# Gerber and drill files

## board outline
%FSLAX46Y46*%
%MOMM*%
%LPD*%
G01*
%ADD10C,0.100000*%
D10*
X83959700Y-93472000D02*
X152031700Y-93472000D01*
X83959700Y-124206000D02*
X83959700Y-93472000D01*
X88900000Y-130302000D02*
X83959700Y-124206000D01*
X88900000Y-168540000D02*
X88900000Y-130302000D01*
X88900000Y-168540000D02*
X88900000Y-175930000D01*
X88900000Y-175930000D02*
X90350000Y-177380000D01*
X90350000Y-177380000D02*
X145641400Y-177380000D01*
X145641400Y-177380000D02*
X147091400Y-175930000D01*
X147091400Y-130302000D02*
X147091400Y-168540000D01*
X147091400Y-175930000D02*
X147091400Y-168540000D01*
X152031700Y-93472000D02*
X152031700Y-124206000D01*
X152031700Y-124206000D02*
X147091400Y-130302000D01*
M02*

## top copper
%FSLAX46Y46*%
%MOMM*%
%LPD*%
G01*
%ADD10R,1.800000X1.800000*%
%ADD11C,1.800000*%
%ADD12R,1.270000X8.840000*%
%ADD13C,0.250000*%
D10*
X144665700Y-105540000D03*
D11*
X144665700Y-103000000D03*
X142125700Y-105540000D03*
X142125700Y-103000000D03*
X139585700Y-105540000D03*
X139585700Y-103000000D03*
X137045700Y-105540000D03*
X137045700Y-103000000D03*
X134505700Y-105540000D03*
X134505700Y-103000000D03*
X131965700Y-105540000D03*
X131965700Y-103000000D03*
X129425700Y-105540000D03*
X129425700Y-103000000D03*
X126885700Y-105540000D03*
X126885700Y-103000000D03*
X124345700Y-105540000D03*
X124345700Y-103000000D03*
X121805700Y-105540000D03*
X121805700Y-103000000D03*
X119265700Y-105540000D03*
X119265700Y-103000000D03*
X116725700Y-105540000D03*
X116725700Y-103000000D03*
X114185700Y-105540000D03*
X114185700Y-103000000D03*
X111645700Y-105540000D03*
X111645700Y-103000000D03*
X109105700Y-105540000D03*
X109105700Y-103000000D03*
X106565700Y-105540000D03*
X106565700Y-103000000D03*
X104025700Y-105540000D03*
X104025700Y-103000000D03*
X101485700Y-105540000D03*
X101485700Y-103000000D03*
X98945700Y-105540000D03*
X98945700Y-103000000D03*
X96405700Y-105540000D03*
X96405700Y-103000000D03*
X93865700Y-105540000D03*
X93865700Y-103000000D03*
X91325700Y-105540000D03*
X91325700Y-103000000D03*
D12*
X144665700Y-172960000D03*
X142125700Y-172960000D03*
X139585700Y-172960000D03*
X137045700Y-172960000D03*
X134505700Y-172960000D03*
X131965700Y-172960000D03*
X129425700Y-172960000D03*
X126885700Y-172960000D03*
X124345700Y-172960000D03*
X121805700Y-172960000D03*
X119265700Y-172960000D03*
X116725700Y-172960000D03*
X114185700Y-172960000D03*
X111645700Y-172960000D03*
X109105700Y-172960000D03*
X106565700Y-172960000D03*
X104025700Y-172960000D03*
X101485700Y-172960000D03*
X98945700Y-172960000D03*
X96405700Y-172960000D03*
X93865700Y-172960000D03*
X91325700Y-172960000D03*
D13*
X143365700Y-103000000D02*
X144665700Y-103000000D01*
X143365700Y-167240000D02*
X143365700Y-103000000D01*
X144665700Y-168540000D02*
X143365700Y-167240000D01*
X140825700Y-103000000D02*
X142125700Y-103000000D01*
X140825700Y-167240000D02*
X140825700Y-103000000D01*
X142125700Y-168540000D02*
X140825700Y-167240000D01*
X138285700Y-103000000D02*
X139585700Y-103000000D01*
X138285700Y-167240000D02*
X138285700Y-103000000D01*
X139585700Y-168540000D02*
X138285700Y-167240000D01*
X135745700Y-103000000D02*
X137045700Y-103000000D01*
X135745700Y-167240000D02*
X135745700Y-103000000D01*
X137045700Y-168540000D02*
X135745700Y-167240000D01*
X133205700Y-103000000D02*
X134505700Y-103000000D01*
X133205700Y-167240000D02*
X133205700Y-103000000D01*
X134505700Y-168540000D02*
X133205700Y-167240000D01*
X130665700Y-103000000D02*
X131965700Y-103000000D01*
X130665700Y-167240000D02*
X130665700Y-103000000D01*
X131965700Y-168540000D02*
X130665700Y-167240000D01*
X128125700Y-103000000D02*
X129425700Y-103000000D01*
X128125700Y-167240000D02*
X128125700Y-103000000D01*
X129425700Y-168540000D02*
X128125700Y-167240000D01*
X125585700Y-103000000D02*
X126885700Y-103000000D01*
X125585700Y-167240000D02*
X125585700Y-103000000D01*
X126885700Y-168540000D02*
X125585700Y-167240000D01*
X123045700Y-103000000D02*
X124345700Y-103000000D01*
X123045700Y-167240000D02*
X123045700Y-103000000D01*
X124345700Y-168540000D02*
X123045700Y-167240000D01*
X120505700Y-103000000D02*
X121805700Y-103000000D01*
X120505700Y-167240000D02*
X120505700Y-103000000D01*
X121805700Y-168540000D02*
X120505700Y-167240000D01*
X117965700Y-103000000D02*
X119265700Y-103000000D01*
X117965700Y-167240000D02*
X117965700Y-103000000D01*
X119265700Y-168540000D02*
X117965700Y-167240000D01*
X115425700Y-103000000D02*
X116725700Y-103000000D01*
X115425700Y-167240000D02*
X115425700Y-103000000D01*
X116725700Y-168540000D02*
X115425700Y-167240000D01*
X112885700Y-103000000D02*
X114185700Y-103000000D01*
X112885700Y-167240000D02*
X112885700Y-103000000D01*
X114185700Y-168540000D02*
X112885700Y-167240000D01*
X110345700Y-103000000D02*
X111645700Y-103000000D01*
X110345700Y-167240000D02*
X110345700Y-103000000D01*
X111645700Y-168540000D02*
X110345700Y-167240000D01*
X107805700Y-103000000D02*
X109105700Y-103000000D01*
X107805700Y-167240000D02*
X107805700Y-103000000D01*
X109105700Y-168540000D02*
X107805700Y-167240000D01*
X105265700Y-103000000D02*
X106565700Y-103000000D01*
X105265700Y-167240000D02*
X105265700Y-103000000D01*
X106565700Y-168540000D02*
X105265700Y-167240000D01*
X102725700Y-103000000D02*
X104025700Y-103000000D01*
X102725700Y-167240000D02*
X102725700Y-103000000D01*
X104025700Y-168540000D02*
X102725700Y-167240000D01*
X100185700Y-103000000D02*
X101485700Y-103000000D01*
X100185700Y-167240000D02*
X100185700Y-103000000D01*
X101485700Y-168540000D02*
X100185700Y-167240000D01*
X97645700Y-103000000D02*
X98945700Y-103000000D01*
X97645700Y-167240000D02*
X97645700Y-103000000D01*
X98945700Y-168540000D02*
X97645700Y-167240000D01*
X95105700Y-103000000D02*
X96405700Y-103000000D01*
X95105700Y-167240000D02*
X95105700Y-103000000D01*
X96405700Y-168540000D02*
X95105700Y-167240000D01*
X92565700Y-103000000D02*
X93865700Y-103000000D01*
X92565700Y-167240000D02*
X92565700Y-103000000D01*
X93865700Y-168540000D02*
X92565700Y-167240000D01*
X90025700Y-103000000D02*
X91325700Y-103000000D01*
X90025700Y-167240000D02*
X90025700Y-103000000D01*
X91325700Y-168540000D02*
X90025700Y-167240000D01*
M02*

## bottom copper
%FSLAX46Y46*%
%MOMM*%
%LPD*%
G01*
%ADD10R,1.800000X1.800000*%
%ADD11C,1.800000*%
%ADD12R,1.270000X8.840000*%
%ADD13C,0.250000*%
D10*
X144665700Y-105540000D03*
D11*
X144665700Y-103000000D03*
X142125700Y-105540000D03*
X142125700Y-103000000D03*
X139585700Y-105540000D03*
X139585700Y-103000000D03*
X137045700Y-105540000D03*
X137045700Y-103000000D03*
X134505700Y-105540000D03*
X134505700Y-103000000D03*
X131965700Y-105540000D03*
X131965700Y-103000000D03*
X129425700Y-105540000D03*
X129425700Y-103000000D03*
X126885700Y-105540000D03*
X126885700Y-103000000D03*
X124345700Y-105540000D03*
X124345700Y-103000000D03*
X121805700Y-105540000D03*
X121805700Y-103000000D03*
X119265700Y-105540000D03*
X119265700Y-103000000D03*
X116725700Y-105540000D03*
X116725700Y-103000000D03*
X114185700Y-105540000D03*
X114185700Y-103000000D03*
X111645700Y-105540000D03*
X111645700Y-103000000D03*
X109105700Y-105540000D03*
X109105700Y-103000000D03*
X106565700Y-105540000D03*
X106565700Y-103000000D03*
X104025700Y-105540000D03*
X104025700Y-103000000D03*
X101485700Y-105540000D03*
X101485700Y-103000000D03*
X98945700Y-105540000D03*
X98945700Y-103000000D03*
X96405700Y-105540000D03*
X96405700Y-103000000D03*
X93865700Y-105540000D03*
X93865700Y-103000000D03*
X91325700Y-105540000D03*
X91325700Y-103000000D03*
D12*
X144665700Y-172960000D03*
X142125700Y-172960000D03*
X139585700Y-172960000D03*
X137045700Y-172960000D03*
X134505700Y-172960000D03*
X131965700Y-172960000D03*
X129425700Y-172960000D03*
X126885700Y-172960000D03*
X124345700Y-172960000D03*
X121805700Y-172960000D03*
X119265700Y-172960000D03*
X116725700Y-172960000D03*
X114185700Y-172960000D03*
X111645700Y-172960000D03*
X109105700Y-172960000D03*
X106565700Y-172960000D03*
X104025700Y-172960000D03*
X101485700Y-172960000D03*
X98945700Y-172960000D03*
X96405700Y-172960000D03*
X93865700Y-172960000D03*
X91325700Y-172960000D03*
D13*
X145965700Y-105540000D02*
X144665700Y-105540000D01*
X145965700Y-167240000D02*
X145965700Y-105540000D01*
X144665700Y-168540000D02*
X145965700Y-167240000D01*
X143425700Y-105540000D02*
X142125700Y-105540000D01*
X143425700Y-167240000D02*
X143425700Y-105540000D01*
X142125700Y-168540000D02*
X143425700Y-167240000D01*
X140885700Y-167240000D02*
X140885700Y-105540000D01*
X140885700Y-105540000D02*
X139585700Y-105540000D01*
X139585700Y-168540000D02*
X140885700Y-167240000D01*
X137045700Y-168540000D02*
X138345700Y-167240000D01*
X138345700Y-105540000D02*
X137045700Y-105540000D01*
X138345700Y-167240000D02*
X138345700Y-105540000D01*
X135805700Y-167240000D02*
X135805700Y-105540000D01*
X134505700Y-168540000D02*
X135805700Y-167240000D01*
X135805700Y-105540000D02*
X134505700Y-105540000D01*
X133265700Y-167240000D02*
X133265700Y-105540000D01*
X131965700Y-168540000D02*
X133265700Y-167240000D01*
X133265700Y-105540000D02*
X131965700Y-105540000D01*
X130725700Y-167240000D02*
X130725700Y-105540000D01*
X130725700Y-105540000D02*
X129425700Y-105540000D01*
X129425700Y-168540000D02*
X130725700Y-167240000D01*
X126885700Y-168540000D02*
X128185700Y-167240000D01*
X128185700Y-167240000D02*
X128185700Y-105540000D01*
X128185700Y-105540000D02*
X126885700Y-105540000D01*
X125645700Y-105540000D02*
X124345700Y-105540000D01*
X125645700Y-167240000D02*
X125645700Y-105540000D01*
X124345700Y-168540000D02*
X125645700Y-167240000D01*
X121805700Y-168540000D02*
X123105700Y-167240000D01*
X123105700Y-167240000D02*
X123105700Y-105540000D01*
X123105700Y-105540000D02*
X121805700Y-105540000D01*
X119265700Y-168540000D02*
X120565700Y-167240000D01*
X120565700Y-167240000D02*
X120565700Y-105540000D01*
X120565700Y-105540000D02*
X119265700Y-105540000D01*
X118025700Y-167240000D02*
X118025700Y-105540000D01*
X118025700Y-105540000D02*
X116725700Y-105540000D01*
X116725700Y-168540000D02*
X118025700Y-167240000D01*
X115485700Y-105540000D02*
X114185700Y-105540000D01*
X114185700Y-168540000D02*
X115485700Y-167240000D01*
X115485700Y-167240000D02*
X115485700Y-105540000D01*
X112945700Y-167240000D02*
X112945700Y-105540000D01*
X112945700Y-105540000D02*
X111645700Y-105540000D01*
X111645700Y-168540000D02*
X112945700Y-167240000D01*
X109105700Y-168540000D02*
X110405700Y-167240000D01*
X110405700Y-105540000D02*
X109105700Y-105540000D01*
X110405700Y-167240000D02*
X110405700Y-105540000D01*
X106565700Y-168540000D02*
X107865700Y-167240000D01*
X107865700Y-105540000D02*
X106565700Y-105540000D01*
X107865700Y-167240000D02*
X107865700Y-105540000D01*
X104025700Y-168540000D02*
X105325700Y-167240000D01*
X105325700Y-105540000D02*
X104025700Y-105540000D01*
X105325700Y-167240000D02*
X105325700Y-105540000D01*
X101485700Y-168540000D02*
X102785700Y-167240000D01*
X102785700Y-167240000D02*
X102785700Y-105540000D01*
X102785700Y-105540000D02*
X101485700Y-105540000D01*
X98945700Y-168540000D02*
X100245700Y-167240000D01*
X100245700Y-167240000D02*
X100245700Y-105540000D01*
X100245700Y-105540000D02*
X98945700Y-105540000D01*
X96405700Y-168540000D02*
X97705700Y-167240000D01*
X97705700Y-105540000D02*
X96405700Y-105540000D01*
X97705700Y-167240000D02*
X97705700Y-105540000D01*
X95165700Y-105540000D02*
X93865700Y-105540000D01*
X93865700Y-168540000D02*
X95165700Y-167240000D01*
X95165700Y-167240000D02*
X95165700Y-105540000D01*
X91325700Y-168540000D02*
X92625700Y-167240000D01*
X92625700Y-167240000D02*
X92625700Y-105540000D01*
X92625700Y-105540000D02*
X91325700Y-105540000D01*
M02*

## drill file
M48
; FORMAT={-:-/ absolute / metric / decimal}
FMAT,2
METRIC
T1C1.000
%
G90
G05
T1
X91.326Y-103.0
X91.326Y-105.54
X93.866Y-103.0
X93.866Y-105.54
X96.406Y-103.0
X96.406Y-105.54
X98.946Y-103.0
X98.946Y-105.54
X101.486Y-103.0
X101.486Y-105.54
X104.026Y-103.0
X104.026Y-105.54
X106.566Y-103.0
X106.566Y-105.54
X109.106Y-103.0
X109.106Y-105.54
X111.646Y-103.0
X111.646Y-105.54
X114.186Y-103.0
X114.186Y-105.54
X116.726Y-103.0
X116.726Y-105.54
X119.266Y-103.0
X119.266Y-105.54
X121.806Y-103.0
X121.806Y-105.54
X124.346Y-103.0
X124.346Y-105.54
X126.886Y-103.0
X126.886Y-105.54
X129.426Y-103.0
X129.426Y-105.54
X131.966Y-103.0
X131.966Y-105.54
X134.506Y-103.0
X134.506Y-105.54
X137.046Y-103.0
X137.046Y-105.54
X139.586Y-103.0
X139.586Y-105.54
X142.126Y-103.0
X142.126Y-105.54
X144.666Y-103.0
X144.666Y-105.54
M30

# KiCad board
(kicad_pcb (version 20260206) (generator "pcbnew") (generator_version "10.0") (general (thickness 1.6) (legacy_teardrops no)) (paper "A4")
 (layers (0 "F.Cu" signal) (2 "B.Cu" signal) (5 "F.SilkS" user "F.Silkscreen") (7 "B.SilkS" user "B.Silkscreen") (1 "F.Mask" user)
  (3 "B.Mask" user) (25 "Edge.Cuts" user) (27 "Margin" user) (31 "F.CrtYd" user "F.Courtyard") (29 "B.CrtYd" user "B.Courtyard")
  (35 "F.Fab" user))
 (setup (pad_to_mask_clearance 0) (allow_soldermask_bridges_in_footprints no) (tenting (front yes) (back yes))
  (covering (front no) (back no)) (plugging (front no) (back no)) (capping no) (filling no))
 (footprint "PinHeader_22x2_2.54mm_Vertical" (layer "F.Cu") (at 0 0)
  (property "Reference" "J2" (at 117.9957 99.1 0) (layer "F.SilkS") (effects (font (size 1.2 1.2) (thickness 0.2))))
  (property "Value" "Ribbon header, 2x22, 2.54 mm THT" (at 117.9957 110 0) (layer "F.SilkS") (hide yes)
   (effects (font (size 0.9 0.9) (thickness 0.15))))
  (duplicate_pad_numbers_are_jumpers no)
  (pad "1" thru_hole rect (at 144.6657 105.54) (size 1.8 1.8) (drill 1) (layers "*.Cu" "*.Mask") (remove_unused_layers no) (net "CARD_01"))
  (pad "2" thru_hole circle (at 144.6657 103) (size 1.8 1.8) (drill 1) (layers "*.Cu" "*.Mask") (remove_unused_layers no) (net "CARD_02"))
  (pad "3" thru_hole circle (at 142.1257 105.54) (size 1.8 1.8) (drill 1) (layers "*.Cu" "*.Mask") (remove_unused_layers no) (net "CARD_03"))
  (pad "4" thru_hole circle (at 142.1257 103) (size 1.8 1.8) (drill 1) (layers "*.Cu" "*.Mask") (remove_unused_layers no) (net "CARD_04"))
  (pad "5" thru_hole circle (at 139.5857 105.54) (size 1.8 1.8) (drill 1) (layers "*.Cu" "*.Mask") (remove_unused_layers no) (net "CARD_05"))
  (pad "6" thru_hole circle (at 139.5857 103) (size 1.8 1.8) (drill 1) (layers "*.Cu" "*.Mask") (remove_unused_layers no) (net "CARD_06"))
  (pad "7" thru_hole circle (at 137.0457 105.54) (size 1.8 1.8) (drill 1) (layers "*.Cu" "*.Mask") (remove_unused_layers no) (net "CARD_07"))
  (pad "8" thru_hole circle (at 137.0457 103) (size 1.8 1.8) (drill 1) (layers "*.Cu" "*.Mask") (remove_unused_layers no) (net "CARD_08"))
  (pad "9" thru_hole circle (at 134.5057 105.54) (size 1.8 1.8) (drill 1) (layers "*.Cu" "*.Mask") (remove_unused_layers no) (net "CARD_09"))
  (pad "10" thru_hole circle (at 134.5057 103) (size 1.8 1.8) (drill 1) (layers "*.Cu" "*.Mask") (remove_unused_layers no) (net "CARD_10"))
  (pad "11" thru_hole circle (at 131.9657 105.54) (size 1.8 1.8) (drill 1) (layers "*.Cu" "*.Mask") (remove_unused_layers no)
   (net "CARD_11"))
  (pad "12" thru_hole circle (at 131.9657 103) (size 1.8 1.8) (drill 1) (layers "*.Cu" "*.Mask") (remove_unused_layers no) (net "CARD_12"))
  (pad "13" thru_hole circle (at 129.4257 105.54) (size 1.8 1.8) (drill 1) (layers "*.Cu" "*.Mask") (remove_unused_layers no)
   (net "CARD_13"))
  (pad "14" thru_hole circle (at 129.4257 103) (size 1.8 1.8) (drill 1) (layers "*.Cu" "*.Mask") (remove_unused_layers no) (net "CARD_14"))
  (pad "15" thru_hole circle (at 126.8857 105.54) (size 1.8 1.8) (drill 1) (layers "*.Cu" "*.Mask") (remove_unused_layers no)
   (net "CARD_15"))
  (pad "16" thru_hole circle (at 126.8857 103) (size 1.8 1.8) (drill 1) (layers "*.Cu" "*.Mask") (remove_unused_layers no) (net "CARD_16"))
  (pad "17" thru_hole circle (at 124.3457 105.54) (size 1.8 1.8) (drill 1) (layers "*.Cu" "*.Mask") (remove_unused_layers no)
   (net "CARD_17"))
  (pad "18" thru_hole circle (at 124.3457 103) (size 1.8 1.8) (drill 1) (layers "*.Cu" "*.Mask") (remove_unused_layers no) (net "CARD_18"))
  (pad "19" thru_hole circle (at 121.8057 105.54) (size 1.8 1.8) (drill 1) (layers "*.Cu" "*.Mask") (remove_unused_layers no)
   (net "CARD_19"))
  (pad "20" thru_hole circle (at 121.8057 103) (size 1.8 1.8) (drill 1) (layers "*.Cu" "*.Mask") (remove_unused_layers no) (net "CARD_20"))
  (pad "21" thru_hole circle (at 119.2657 105.54) (size 1.8 1.8) (drill 1) (layers "*.Cu" "*.Mask") (remove_unused_layers no)
   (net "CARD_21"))
  (pad "22" thru_hole circle (at 119.2657 103) (size 1.8 1.8) (drill 1) (layers "*.Cu" "*.Mask") (remove_unused_layers no) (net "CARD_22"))
  (pad "23" thru_hole circle (at 116.7257 105.54) (size 1.8 1.8) (drill 1) (layers "*.Cu" "*.Mask") (remove_unused_layers no)
   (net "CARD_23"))
  (pad "24" thru_hole circle (at 116.7257 103) (size 1.8 1.8) (drill 1) (layers "*.Cu" "*.Mask") (remove_unused_layers no) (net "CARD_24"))
  (pad "25" thru_hole circle (at 114.1857 105.54) (size 1.8 1.8) (drill 1) (layers "*.Cu" "*.Mask") (remove_unused_layers no)
   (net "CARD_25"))
  (pad "26" thru_hole circle (at 114.1857 103) (size 1.8 1.8) (drill 1) (layers "*.Cu" "*.Mask") (remove_unused_layers no) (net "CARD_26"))
  (pad "27" thru_hole circle (at 111.6457 105.54) (size 1.8 1.8) (drill 1) (layers "*.Cu" "*.Mask") (remove_unused_layers no)
   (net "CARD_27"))
  (pad "28" thru_hole circle (at 111.6457 103) (size 1.8 1.8) (drill 1) (layers "*.Cu" "*.Mask") (remove_unused_layers no) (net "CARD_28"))
  (pad "29" thru_hole circle (at 109.1057 105.54) (size 1.8 1.8) (drill 1) (layers "*.Cu" "*.Mask") (remove_unused_layers no)
   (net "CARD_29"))
  (pad "30" thru_hole circle (at 109.1057 103) (size 1.8 1.8) (drill 1) (layers "*.Cu" "*.Mask") (remove_unused_layers no) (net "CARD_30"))
  (pad "31" thru_hole circle (at 106.5657 105.54) (size 1.8 1.8) (drill 1) (layers "*.Cu" "*.Mask") (remove_unused_layers no)
   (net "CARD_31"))
  (pad "32" thru_hole circle (at 106.5657 103) (size 1.8 1.8) (drill 1) (layers "*.Cu" "*.Mask") (remove_unused_layers no) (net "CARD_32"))
  (pad "33" thru_hole circle (at 104.0257 105.54) (size 1.8 1.8) (drill 1) (layers "*.Cu" "*.Mask") (remove_unused_layers no)
   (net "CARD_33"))
  (pad "34" thru_hole circle (at 104.0257 103) (size 1.8 1.8) (drill 1) (layers "*.Cu" "*.Mask") (remove_unused_layers no) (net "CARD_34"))
  (pad "35" thru_hole circle (at 101.4857 105.54) (size 1.8 1.8) (drill 1) (layers "*.Cu" "*.Mask") (remove_unused_layers no)
   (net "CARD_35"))
  (pad "36" thru_hole circle (at 101.4857 103) (size 1.8 1.8) (drill 1) (layers "*.Cu" "*.Mask") (remove_unused_layers no) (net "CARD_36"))
  (pad "37" thru_hole circle (at 98.9457 105.54) (size 1.8 1.8) (drill 1) (layers "*.Cu" "*.Mask") (remove_unused_layers no) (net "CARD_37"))
  (pad "38" thru_hole circle (at 98.9457 103) (size 1.8 1.8) (drill 1) (layers "*.Cu" "*.Mask") (remove_unused_layers no) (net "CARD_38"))
  (pad "39" thru_hole circle (at 96.4057 105.54) (size 1.8 1.8) (drill 1) (layers "*.Cu" "*.Mask") (remove_unused_layers no) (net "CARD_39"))
  (pad "40" thru_hole circle (at 96.4057 103) (size 1.8 1.8) (drill 1) (layers "*.Cu" "*.Mask") (remove_unused_layers no) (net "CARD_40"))
  (pad "41" thru_hole circle (at 93.8657 105.54) (size 1.8 1.8) (drill 1) (layers "*.Cu" "*.Mask") (remove_unused_layers no) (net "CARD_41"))
  (pad "42" thru_hole circle (at 93.8657 103) (size 1.8 1.8) (drill 1) (layers "*.Cu" "*.Mask") (remove_unused_layers no) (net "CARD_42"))
  (pad "43" thru_hole circle (at 91.3257 105.54) (size 1.8 1.8) (drill 1) (layers "*.Cu" "*.Mask") (remove_unused_layers no) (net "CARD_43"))
  (pad "44" thru_hole circle (at 91.3257 103) (size 1.8 1.8) (drill 1) (layers "*.Cu" "*.Mask") (remove_unused_layers no) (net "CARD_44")))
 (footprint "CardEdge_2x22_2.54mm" (layer "F.Cu") (at 0 -15)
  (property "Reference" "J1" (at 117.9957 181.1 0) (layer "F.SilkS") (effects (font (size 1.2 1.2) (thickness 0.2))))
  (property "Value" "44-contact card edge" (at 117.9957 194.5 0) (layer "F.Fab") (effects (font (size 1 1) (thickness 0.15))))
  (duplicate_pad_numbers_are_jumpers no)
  (pad "1" connect rect (at 144.6657 187.96) (size 1.27 8.84) (layers "B.Cu" "B.Mask") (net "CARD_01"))
  (pad "2" connect rect (at 144.6657 187.96) (size 1.27 8.84) (layers "F.Cu" "F.Mask") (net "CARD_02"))
  (pad "3" connect rect (at 142.1257 187.96) (size 1.27 8.84) (layers "B.Cu" "B.Mask") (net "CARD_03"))
  (pad "4" connect rect (at 142.1257 187.96) (size 1.27 8.84) (layers "F.Cu" "F.Mask") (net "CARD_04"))
  (pad "5" connect rect (at 139.5857 187.96) (size 1.27 8.84) (layers "B.Cu" "B.Mask") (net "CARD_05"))
  (pad "6" connect rect (at 139.5857 187.96) (size 1.27 8.84) (layers "F.Cu" "F.Mask") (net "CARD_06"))
  (pad "7" connect rect (at 137.0457 187.96) (size 1.27 8.84) (layers "B.Cu" "B.Mask") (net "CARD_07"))
  (pad "8" connect rect (at 137.0457 187.96) (size 1.27 8.84) (layers "F.Cu" "F.Mask") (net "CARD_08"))
  (pad "9" connect rect (at 134.5057 187.96) (size 1.27 8.84) (layers "B.Cu" "B.Mask") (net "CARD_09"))
  (pad "10" connect rect (at 134.5057 187.96) (size 1.27 8.84) (layers "F.Cu" "F.Mask") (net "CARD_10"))
  (pad "11" connect rect (at 131.9657 187.96) (size 1.27 8.84) (layers "B.Cu" "B.Mask") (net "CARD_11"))
  (pad "12" connect rect (at 131.9657 187.96) (size 1.27 8.84) (layers "F.Cu" "F.Mask") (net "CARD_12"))
  (pad "13" connect rect (at 129.4257 187.96) (size 1.27 8.84) (layers "B.Cu" "B.Mask") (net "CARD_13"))
  (pad "14" connect rect (at 129.4257 187.96) (size 1.27 8.84) (layers "F.Cu" "F.Mask") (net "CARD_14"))
  (pad "15" connect rect (at 126.8857 187.96) (size 1.27 8.84) (layers "B.Cu" "B.Mask") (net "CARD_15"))
  (pad "16" connect rect (at 126.8857 187.96) (size 1.27 8.84) (layers "F.Cu" "F.Mask") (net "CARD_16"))
  (pad "17" connect rect (at 124.3457 187.96) (size 1.27 8.84) (layers "B.Cu" "B.Mask") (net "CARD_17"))
  (pad "18" connect rect (at 124.3457 187.96) (size 1.27 8.84) (layers "F.Cu" "F.Mask") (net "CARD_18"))
  (pad "19" connect rect (at 121.8057 187.96) (size 1.27 8.84) (layers "B.Cu" "B.Mask") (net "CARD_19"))
  (pad "20" connect rect (at 121.8057 187.96) (size 1.27 8.84) (layers "F.Cu" "F.Mask") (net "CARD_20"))
  (pad "21" connect rect (at 119.2657 187.96) (size 1.27 8.84) (layers "B.Cu" "B.Mask") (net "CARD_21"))
  (pad "22" connect rect (at 119.2657 187.96) (size 1.27 8.84) (layers "F.Cu" "F.Mask") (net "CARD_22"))
  (pad "23" connect rect (at 116.7257 187.96) (size 1.27 8.84) (layers "B.Cu" "B.Mask") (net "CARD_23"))
  (pad "24" connect rect (at 116.7257 187.96) (size 1.27 8.84) (layers "F.Cu" "F.Mask") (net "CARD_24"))
  (pad "25" connect rect (at 114.1857 187.96) (size 1.27 8.84) (layers "B.Cu" "B.Mask") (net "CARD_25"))
  (pad "26" connect rect (at 114.1857 187.96) (size 1.27 8.84) (layers "F.Cu" "F.Mask") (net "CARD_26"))
  (pad "27" connect rect (at 111.6457 187.96) (size 1.27 8.84) (layers "B.Cu" "B.Mask") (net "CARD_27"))
  (pad "28" connect rect (at 111.6457 187.96) (size 1.27 8.84) (layers "F.Cu" "F.Mask") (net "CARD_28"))
  (pad "29" connect rect (at 109.1057 187.96) (size 1.27 8.84) (layers "B.Cu" "B.Mask") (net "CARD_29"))
  (pad "30" connect rect (at 109.1057 187.96) (size 1.27 8.84) (layers "F.Cu" "F.Mask") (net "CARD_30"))
  (pad "31" connect rect (at 106.5657 187.96) (size 1.27 8.84) (layers "B.Cu" "B.Mask") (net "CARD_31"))
  (pad "32" connect rect (at 106.5657 187.96) (size 1.27 8.84) (layers "F.Cu" "F.Mask") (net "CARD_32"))
  (pad "33" connect rect (at 104.0257 187.96) (size 1.27 8.84) (layers "B.Cu" "B.Mask") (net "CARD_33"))
  (pad "34" connect rect (at 104.0257 187.96) (size 1.27 8.84) (layers "F.Cu" "F.Mask") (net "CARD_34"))
  (pad "35" connect rect (at 101.4857 187.96) (size 1.27 8.84) (layers "B.Cu" "B.Mask") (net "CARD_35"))
  (pad "36" connect rect (at 101.4857 187.96) (size 1.27 8.84) (layers "F.Cu" "F.Mask") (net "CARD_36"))
  (pad "37" connect rect (at 98.9457 187.96) (size 1.27 8.84) (layers "B.Cu" "B.Mask") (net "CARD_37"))
  (pad "38" connect rect (at 98.9457 187.96) (size 1.27 8.84) (layers "F.Cu" "F.Mask") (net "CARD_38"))
  (pad "39" connect rect (at 96.4057 187.96) (size 1.27 8.84) (layers "B.Cu" "B.Mask") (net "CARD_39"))
  (pad "40" connect rect (at 96.4057 187.96) (size 1.27 8.84) (layers "F.Cu" "F.Mask") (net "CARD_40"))
  (pad "41" connect rect (at 93.8657 187.96) (size 1.27 8.84) (layers "B.Cu" "B.Mask") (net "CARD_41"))
  (pad "42" connect rect (at 93.8657 187.96) (size 1.27 8.84) (layers "F.Cu" "F.Mask") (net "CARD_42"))
  (pad "43" connect rect (at 91.3257 187.96) (size 1.27 8.84) (layers "B.Cu" "B.Mask") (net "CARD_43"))
  (pad "44" connect rect (at 91.3257 187.96) (size 1.27 8.84) (layers "F.Cu" "F.Mask") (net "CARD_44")))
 (gr_line (start 83.9597 93.472) (end 152.0317 93.472) (stroke (width 0.1) (type solid)) (layer "Edge.Cuts"))
 (gr_line (start 83.9597 124.206) (end 83.9597 93.472) (stroke (width 0.1) (type solid)) (layer "Edge.Cuts"))
 (gr_line (start 88.9 130.302) (end 83.9597 124.206) (stroke (width 0.1) (type solid)) (layer "Edge.Cuts"))
 (gr_line (start 88.9 168.54) (end 88.9 130.302) (stroke (width 0.1) (type solid)) (layer "Edge.Cuts"))
 (gr_line (start 88.9 168.54) (end 88.9 175.93) (stroke (width 0.1) (type solid)) (layer "Edge.Cuts"))
 (gr_line (start 88.9 175.93) (end 90.35 177.38) (stroke (width 0.1) (type solid)) (layer "Edge.Cuts"))
 (gr_line (start 90.35 177.38) (end 145.6414 177.38) (stroke (width 0.1) (type solid)) (layer "Edge.Cuts"))
 (gr_line (start 145.6414 177.38) (end 147.0914 175.93) (stroke (width 0.1) (type solid)) (layer "Edge.Cuts"))
 (gr_line (start 147.0914 130.302) (end 147.0914 168.54) (stroke (width 0.1) (type solid)) (layer "Edge.Cuts"))
 (gr_line (start 147.0914 175.93) (end 147.0914 168.54) (stroke (width 0.1) (type solid)) (layer "Edge.Cuts"))
 (gr_line (start 152.0317 93.472) (end 152.0317 124.206) (stroke (width 0.1) (type solid)) (layer "Edge.Cuts"))
 (gr_line (start 152.0317 124.206) (end 147.0914 130.302) (stroke (width 0.1) (type solid)) (layer "Edge.Cuts"))
 (segment (start 145.9657 105.54) (end 144.6657 105.54) (width 0.25) (layer "B.Cu") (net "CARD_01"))
 (segment (start 145.9657 167.24) (end 145.9657 105.54) (width 0.25) (layer "B.Cu") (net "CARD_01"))
 (segment (start 144.6657 168.54) (end 145.9657 167.24) (width 0.25) (layer "B.Cu") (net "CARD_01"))
 (segment (start 143.3657 103) (end 144.6657 103) (width 0.25) (layer "F.Cu") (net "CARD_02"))
 (segment (start 143.3657 167.24) (end 143.3657 103) (width 0.25) (layer "F.Cu") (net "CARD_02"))
 (segment (start 144.6657 168.54) (end 143.3657 167.24) (width 0.25) (layer "F.Cu") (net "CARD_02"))
 (segment (start 143.4257 105.54) (end 142.1257 105.54) (width 0.25) (layer "B.Cu") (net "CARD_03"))
 (segment (start 143.4257 167.24) (end 143.4257 105.54) (width 0.25) (layer "B.Cu") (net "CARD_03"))
 (segment (start 142.1257 168.54) (end 143.4257 167.24) (width 0.25) (layer "B.Cu") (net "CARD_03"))
 (segment (start 140.8257 103) (end 142.1257 103) (width 0.25) (layer "F.Cu") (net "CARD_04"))
 (segment (start 140.8257 167.24) (end 140.8257 103) (width 0.25) (layer "F.Cu") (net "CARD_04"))
 (segment (start 142.1257 168.54) (end 140.8257 167.24) (width 0.25) (layer "F.Cu") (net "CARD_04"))
 (segment (start 140.8857 167.24) (end 140.8857 105.54) (width 0.25) (layer "B.Cu") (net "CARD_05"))
 (segment (start 140.8857 105.54) (end 139.5857 105.54) (width 0.25) (layer "B.Cu") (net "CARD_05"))
 (segment (start 139.5857 168.54) (end 140.8857 167.24) (width 0.25) (layer "B.Cu") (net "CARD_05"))
 (segment (start 138.2857 103) (end 139.5857 103) (width 0.25) (layer "F.Cu") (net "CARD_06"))
 (segment (start 138.2857 167.24) (end 138.2857 103) (width 0.25) (layer "F.Cu") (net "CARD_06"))
 (segment (start 139.5857 168.54) (end 138.2857 167.24) (width 0.25) (layer "F.Cu") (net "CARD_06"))
 (segment (start 137.0457 168.54) (end 138.3457 167.24) (width 0.25) (layer "B.Cu") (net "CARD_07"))
 (segment (start 138.3457 105.54) (end 137.0457 105.54) (width 0.25) (layer "B.Cu") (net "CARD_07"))
 (segment (start 138.3457 167.24) (end 138.3457 105.54) (width 0.25) (layer "B.Cu") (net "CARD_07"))
 (segment (start 135.7457 103) (end 137.0457 103) (width 0.25) (layer "F.Cu") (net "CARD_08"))
 (segment (start 135.7457 167.24) (end 135.7457 103) (width 0.25) (layer "F.Cu") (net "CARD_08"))
 (segment (start 137.0457 168.54) (end 135.7457 167.24) (width 0.25) (layer "F.Cu") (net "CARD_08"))
 (segment (start 135.8057 167.24) (end 135.8057 105.54) (width 0.25) (layer "B.Cu") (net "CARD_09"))
 (segment (start 134.5057 168.54) (end 135.8057 167.24) (width 0.25) (layer "B.Cu") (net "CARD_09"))
 (segment (start 135.8057 105.54) (end 134.5057 105.54) (width 0.25) (layer "B.Cu") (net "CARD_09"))
 (segment (start 133.2057 103) (end 134.5057 103) (width 0.25) (layer "F.Cu") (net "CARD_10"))
 (segment (start 133.2057 167.24) (end 133.2057 103) (width 0.25) (layer "F.Cu") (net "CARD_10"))
 (segment (start 134.5057 168.54) (end 133.2057 167.24) (width 0.25) (layer "F.Cu") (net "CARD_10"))
 (segment (start 133.2657 167.24) (end 133.2657 105.54) (width 0.25) (layer "B.Cu") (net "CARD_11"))
 (segment (start 131.9657 168.54) (end 133.2657 167.24) (width 0.25) (layer "B.Cu") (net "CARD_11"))
 (segment (start 133.2657 105.54) (end 131.9657 105.54) (width 0.25) (layer "B.Cu") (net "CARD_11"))
 (segment (start 130.6657 103) (end 131.9657 103) (width 0.25) (layer "F.Cu") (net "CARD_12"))
 (segment (start 130.6657 167.24) (end 130.6657 103) (width 0.25) (layer "F.Cu") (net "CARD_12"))
 (segment (start 131.9657 168.54) (end 130.6657 167.24) (width 0.25) (layer "F.Cu") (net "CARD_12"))
 (segment (start 130.7257 167.24) (end 130.7257 105.54) (width 0.25) (layer "B.Cu") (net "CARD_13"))
 (segment (start 130.7257 105.54) (end 129.4257 105.54) (width 0.25) (layer "B.Cu") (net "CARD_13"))
 (segment (start 129.4257 168.54) (end 130.7257 167.24) (width 0.25) (layer "B.Cu") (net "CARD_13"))
 (segment (start 128.1257 103) (end 129.4257 103) (width 0.25) (layer "F.Cu") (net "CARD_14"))
 (segment (start 128.1257 167.24) (end 128.1257 103) (width 0.25) (layer "F.Cu") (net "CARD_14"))
 (segment (start 129.4257 168.54) (end 128.1257 167.24) (width 0.25) (layer "F.Cu") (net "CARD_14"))
 (segment (start 126.8857 168.54) (end 128.1857 167.24) (width 0.25) (layer "B.Cu") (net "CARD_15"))
 (segment (start 128.1857 167.24) (end 128.1857 105.54) (width 0.25) (layer "B.Cu") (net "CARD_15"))
 (segment (start 128.1857 105.54) (end 126.8857 105.54) (width 0.25) (layer "B.Cu") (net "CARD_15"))
 (segment (start 125.5857 103) (end 126.8857 103) (width 0.25) (layer "F.Cu") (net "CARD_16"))
 (segment (start 125.5857 167.24) (end 125.5857 103) (width 0.25) (layer "F.Cu") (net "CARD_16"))
 (segment (start 126.8857 168.54) (end 125.5857 167.24) (width 0.25) (layer "F.Cu") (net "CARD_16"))
 (segment (start 125.6457 105.54) (end 124.3457 105.54) (width 0.25) (layer "B.Cu") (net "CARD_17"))
 (segment (start 125.6457 167.24) (end 125.6457 105.54) (width 0.25) (layer "B.Cu") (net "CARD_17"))
 (segment (start 124.3457 168.54) (end 125.6457 167.24) (width 0.25) (layer "B.Cu") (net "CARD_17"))
 (segment (start 123.0457 103) (end 124.3457 103) (width 0.25) (layer "F.Cu") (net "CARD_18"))
 (segment (start 123.0457 167.24) (end 123.0457 103) (width 0.25) (layer "F.Cu") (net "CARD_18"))
 (segment (start 124.3457 168.54) (end 123.0457 167.24) (width 0.25) (layer "F.Cu") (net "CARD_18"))
 (segment (start 121.8057 168.54) (end 123.1057 167.24) (width 0.25) (layer "B.Cu") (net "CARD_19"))
 (segment (start 123.1057 167.24) (end 123.1057 105.54) (width 0.25) (layer "B.Cu") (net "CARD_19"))
 (segment (start 123.1057 105.54) (end 121.8057 105.54) (width 0.25) (layer "B.Cu") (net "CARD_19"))
 (segment (start 120.5057 103) (end 121.8057 103) (width 0.25) (layer "F.Cu") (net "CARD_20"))
 (segment (start 120.5057 167.24) (end 120.5057 103) (width 0.25) (layer "F.Cu") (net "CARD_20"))
 (segment (start 121.8057 168.54) (end 120.5057 167.24) (width 0.25) (layer "F.Cu") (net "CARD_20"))
 (segment (start 119.2657 168.54) (end 120.5657 167.24) (width 0.25) (layer "B.Cu") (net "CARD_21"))
 (segment (start 120.5657 167.24) (end 120.5657 105.54) (width 0.25) (layer "B.Cu") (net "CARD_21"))
 (segment (start 120.5657 105.54) (end 119.2657 105.54) (width 0.25) (layer "B.Cu") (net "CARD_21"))
 (segment (start 117.9657 103) (end 119.2657 103) (width 0.25) (layer "F.Cu") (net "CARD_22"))
 (segment (start 117.9657 167.24) (end 117.9657 103) (width 0.25) (layer "F.Cu") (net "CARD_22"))
 (segment (start 119.2657 168.54) (end 117.9657 167.24) (width 0.25) (layer "F.Cu") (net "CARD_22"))
 (segment (start 118.0257 167.24) (end 118.0257 105.54) (width 0.25) (layer "B.Cu") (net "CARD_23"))
 (segment (start 118.0257 105.54) (end 116.7257 105.54) (width 0.25) (layer "B.Cu") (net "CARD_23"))
 (segment (start 116.7257 168.54) (end 118.0257 167.24) (width 0.25) (layer "B.Cu") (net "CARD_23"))
 (segment (start 115.4257 103) (end 116.7257 103) (width 0.25) (layer "F.Cu") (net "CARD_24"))
 (segment (start 115.4257 167.24) (end 115.4257 103) (width 0.25) (layer "F.Cu") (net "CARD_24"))
 (segment (start 116.7257 168.54) (end 115.4257 167.24) (width 0.25) (layer "F.Cu") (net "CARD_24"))
 (segment (start 115.4857 105.54) (end 114.1857 105.54) (width 0.25) (layer "B.Cu") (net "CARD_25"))
 (segment (start 114.1857 168.54) (end 115.4857 167.24) (width 0.25) (layer "B.Cu") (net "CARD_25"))
 (segment (start 115.4857 167.24) (end 115.4857 105.54) (width 0.25) (layer "B.Cu") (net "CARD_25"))
 (segment (start 112.8857 103) (end 114.1857 103) (width 0.25) (layer "F.Cu") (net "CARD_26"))
 (segment (start 112.8857 167.24) (end 112.8857 103) (width 0.25) (layer "F.Cu") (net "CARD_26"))
 (segment (start 114.1857 168.54) (end 112.8857 167.24) (width 0.25) (layer "F.Cu") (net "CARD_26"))
 (segment (start 112.9457 167.24) (end 112.9457 105.54) (width 0.25) (layer "B.Cu") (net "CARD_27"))
 (segment (start 112.9457 105.54) (end 111.6457 105.54) (width 0.25) (layer "B.Cu") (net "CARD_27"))
 (segment (start 111.6457 168.54) (end 112.9457 167.24) (width 0.25) (layer "B.Cu") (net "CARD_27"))
 (segment (start 110.3457 103) (end 111.6457 103) (width 0.25) (layer "F.Cu") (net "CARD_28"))
 (segment (start 110.3457 167.24) (end 110.3457 103) (width 0.25) (layer "F.Cu") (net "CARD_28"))
 (segment (start 111.6457 168.54) (end 110.3457 167.24) (width 0.25) (layer "F.Cu") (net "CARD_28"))
 (segment (start 109.1057 168.54) (end 110.4057 167.24) (width 0.25) (layer "B.Cu") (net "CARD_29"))
 (segment (start 110.4057 105.54) (end 109.1057 105.54) (width 0.25) (layer "B.Cu") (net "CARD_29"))
 (segment (start 110.4057 167.24) (end 110.4057 105.54) (width 0.25) (layer "B.Cu") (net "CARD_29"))
 (segment (start 107.8057 103) (end 109.1057 103) (width 0.25) (layer "F.Cu") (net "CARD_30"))
 (segment (start 107.8057 167.24) (end 107.8057 103) (width 0.25) (layer "F.Cu") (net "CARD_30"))
 (segment (start 109.1057 168.54) (end 107.8057 167.24) (width 0.25) (layer "F.Cu") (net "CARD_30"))
 (segment (start 106.5657 168.54) (end 107.8657 167.24) (width 0.25) (layer "B.Cu") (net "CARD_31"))
 (segment (start 107.8657 105.54) (end 106.5657 105.54) (width 0.25) (layer "B.Cu") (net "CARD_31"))
 (segment (start 107.8657 167.24) (end 107.8657 105.54) (width 0.25) (layer "B.Cu") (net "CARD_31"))
 (segment (start 105.2657 103) (end 106.5657 103) (width 0.25) (layer "F.Cu") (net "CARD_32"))
 (segment (start 105.2657 167.24) (end 105.2657 103) (width 0.25) (layer "F.Cu") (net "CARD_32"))
 (segment (start 106.5657 168.54) (end 105.2657 167.24) (width 0.25) (layer "F.Cu") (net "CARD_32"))
 (segment (start 104.0257 168.54) (end 105.3257 167.24) (width 0.25) (layer "B.Cu") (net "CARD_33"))
 (segment (start 105.3257 105.54) (end 104.0257 105.54) (width 0.25) (layer "B.Cu") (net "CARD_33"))
 (segment (start 105.3257 167.24) (end 105.3257 105.54) (width 0.25) (layer "B.Cu") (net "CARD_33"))
 (segment (start 102.7257 103) (end 104.0257 103) (width 0.25) (layer "F.Cu") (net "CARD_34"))
 (segment (start 102.7257 167.24) (end 102.7257 103) (width 0.25) (layer "F.Cu") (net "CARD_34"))
 (segment (start 104.0257 168.54) (end 102.7257 167.24) (width 0.25) (layer "F.Cu") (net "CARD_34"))
 (segment (start 101.4857 168.54) (end 102.7857 167.24) (width 0.25) (layer "B.Cu") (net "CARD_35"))
 (segment (start 102.7857 167.24) (end 102.7857 105.54) (width 0.25) (layer "B.Cu") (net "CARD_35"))
 (segment (start 102.7857 105.54) (end 101.4857 105.54) (width 0.25) (layer "B.Cu") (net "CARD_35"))
 (segment (start 100.1857 103) (end 101.4857 103) (width 0.25) (layer "F.Cu") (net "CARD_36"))
 (segment (start 100.1857 167.24) (end 100.1857 103) (width 0.25) (layer "F.Cu") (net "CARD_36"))
 (segment (start 101.4857 168.54) (end 100.1857 167.24) (width 0.25) (layer "F.Cu") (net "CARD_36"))
 (segment (start 98.9457 168.54) (end 100.2457 167.24) (width 0.25) (layer "B.Cu") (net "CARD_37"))
 (segment (start 100.2457 167.24) (end 100.2457 105.54) (width 0.25) (layer "B.Cu") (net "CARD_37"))
 (segment (start 100.2457 105.54) (end 98.9457 105.54) (width 0.25) (layer "B.Cu") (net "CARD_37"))
 (segment (start 97.6457 103) (end 98.9457 103) (width 0.25) (layer "F.Cu") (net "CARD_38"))
 (segment (start 97.6457 167.24) (end 97.6457 103) (width 0.25) (layer "F.Cu") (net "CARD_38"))
 (segment (start 98.9457 168.54) (end 97.6457 167.24) (width 0.25) (layer "F.Cu") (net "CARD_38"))
 (segment (start 96.4057 168.54) (end 97.7057 167.24) (width 0.25) (layer "B.Cu") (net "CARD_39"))
 (segment (start 97.7057 105.54) (end 96.4057 105.54) (width 0.25) (layer "B.Cu") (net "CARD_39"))
 (segment (start 97.7057 167.24) (end 97.7057 105.54) (width 0.25) (layer "B.Cu") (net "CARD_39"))
 (segment (start 95.1057 103) (end 96.4057 103) (width 0.25) (layer "F.Cu") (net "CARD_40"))
 (segment (start 95.1057 167.24) (end 95.1057 103) (width 0.25) (layer "F.Cu") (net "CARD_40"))
 (segment (start 96.4057 168.54) (end 95.1057 167.24) (width 0.25) (layer "F.Cu") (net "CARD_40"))
 (segment (start 95.1657 105.54) (end 93.8657 105.54) (width 0.25) (layer "B.Cu") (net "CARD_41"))
 (segment (start 93.8657 168.54) (end 95.1657 167.24) (width 0.25) (layer "B.Cu") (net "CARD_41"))
 (segment (start 95.1657 167.24) (end 95.1657 105.54) (width 0.25) (layer "B.Cu") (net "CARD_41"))
 (segment (start 92.5657 103) (end 93.8657 103) (width 0.25) (layer "F.Cu") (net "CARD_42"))
 (segment (start 92.5657 167.24) (end 92.5657 103) (width 0.25) (layer "F.Cu") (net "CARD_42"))
 (segment (start 93.8657 168.54) (end 92.5657 167.24) (width 0.25) (layer "F.Cu") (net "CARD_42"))
 (segment (start 91.3257 168.54) (end 92.6257 167.24) (width 0.25) (layer "B.Cu") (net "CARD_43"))
 (segment (start 92.6257 167.24) (end 92.6257 105.54) (width 0.25) (layer "B.Cu") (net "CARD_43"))
 (segment (start 92.6257 105.54) (end 91.3257 105.54) (width 0.25) (layer "B.Cu") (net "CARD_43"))
 (segment (start 90.0257 103) (end 91.3257 103) (width 0.25) (layer "F.Cu") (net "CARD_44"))
 (segment (start 90.0257 167.24) (end 90.0257 103) (width 0.25) (layer "F.Cu") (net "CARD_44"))
 (segment (start 91.3257 168.54) (end 90.0257 167.24) (width 0.25) (layer "F.Cu") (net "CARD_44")))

